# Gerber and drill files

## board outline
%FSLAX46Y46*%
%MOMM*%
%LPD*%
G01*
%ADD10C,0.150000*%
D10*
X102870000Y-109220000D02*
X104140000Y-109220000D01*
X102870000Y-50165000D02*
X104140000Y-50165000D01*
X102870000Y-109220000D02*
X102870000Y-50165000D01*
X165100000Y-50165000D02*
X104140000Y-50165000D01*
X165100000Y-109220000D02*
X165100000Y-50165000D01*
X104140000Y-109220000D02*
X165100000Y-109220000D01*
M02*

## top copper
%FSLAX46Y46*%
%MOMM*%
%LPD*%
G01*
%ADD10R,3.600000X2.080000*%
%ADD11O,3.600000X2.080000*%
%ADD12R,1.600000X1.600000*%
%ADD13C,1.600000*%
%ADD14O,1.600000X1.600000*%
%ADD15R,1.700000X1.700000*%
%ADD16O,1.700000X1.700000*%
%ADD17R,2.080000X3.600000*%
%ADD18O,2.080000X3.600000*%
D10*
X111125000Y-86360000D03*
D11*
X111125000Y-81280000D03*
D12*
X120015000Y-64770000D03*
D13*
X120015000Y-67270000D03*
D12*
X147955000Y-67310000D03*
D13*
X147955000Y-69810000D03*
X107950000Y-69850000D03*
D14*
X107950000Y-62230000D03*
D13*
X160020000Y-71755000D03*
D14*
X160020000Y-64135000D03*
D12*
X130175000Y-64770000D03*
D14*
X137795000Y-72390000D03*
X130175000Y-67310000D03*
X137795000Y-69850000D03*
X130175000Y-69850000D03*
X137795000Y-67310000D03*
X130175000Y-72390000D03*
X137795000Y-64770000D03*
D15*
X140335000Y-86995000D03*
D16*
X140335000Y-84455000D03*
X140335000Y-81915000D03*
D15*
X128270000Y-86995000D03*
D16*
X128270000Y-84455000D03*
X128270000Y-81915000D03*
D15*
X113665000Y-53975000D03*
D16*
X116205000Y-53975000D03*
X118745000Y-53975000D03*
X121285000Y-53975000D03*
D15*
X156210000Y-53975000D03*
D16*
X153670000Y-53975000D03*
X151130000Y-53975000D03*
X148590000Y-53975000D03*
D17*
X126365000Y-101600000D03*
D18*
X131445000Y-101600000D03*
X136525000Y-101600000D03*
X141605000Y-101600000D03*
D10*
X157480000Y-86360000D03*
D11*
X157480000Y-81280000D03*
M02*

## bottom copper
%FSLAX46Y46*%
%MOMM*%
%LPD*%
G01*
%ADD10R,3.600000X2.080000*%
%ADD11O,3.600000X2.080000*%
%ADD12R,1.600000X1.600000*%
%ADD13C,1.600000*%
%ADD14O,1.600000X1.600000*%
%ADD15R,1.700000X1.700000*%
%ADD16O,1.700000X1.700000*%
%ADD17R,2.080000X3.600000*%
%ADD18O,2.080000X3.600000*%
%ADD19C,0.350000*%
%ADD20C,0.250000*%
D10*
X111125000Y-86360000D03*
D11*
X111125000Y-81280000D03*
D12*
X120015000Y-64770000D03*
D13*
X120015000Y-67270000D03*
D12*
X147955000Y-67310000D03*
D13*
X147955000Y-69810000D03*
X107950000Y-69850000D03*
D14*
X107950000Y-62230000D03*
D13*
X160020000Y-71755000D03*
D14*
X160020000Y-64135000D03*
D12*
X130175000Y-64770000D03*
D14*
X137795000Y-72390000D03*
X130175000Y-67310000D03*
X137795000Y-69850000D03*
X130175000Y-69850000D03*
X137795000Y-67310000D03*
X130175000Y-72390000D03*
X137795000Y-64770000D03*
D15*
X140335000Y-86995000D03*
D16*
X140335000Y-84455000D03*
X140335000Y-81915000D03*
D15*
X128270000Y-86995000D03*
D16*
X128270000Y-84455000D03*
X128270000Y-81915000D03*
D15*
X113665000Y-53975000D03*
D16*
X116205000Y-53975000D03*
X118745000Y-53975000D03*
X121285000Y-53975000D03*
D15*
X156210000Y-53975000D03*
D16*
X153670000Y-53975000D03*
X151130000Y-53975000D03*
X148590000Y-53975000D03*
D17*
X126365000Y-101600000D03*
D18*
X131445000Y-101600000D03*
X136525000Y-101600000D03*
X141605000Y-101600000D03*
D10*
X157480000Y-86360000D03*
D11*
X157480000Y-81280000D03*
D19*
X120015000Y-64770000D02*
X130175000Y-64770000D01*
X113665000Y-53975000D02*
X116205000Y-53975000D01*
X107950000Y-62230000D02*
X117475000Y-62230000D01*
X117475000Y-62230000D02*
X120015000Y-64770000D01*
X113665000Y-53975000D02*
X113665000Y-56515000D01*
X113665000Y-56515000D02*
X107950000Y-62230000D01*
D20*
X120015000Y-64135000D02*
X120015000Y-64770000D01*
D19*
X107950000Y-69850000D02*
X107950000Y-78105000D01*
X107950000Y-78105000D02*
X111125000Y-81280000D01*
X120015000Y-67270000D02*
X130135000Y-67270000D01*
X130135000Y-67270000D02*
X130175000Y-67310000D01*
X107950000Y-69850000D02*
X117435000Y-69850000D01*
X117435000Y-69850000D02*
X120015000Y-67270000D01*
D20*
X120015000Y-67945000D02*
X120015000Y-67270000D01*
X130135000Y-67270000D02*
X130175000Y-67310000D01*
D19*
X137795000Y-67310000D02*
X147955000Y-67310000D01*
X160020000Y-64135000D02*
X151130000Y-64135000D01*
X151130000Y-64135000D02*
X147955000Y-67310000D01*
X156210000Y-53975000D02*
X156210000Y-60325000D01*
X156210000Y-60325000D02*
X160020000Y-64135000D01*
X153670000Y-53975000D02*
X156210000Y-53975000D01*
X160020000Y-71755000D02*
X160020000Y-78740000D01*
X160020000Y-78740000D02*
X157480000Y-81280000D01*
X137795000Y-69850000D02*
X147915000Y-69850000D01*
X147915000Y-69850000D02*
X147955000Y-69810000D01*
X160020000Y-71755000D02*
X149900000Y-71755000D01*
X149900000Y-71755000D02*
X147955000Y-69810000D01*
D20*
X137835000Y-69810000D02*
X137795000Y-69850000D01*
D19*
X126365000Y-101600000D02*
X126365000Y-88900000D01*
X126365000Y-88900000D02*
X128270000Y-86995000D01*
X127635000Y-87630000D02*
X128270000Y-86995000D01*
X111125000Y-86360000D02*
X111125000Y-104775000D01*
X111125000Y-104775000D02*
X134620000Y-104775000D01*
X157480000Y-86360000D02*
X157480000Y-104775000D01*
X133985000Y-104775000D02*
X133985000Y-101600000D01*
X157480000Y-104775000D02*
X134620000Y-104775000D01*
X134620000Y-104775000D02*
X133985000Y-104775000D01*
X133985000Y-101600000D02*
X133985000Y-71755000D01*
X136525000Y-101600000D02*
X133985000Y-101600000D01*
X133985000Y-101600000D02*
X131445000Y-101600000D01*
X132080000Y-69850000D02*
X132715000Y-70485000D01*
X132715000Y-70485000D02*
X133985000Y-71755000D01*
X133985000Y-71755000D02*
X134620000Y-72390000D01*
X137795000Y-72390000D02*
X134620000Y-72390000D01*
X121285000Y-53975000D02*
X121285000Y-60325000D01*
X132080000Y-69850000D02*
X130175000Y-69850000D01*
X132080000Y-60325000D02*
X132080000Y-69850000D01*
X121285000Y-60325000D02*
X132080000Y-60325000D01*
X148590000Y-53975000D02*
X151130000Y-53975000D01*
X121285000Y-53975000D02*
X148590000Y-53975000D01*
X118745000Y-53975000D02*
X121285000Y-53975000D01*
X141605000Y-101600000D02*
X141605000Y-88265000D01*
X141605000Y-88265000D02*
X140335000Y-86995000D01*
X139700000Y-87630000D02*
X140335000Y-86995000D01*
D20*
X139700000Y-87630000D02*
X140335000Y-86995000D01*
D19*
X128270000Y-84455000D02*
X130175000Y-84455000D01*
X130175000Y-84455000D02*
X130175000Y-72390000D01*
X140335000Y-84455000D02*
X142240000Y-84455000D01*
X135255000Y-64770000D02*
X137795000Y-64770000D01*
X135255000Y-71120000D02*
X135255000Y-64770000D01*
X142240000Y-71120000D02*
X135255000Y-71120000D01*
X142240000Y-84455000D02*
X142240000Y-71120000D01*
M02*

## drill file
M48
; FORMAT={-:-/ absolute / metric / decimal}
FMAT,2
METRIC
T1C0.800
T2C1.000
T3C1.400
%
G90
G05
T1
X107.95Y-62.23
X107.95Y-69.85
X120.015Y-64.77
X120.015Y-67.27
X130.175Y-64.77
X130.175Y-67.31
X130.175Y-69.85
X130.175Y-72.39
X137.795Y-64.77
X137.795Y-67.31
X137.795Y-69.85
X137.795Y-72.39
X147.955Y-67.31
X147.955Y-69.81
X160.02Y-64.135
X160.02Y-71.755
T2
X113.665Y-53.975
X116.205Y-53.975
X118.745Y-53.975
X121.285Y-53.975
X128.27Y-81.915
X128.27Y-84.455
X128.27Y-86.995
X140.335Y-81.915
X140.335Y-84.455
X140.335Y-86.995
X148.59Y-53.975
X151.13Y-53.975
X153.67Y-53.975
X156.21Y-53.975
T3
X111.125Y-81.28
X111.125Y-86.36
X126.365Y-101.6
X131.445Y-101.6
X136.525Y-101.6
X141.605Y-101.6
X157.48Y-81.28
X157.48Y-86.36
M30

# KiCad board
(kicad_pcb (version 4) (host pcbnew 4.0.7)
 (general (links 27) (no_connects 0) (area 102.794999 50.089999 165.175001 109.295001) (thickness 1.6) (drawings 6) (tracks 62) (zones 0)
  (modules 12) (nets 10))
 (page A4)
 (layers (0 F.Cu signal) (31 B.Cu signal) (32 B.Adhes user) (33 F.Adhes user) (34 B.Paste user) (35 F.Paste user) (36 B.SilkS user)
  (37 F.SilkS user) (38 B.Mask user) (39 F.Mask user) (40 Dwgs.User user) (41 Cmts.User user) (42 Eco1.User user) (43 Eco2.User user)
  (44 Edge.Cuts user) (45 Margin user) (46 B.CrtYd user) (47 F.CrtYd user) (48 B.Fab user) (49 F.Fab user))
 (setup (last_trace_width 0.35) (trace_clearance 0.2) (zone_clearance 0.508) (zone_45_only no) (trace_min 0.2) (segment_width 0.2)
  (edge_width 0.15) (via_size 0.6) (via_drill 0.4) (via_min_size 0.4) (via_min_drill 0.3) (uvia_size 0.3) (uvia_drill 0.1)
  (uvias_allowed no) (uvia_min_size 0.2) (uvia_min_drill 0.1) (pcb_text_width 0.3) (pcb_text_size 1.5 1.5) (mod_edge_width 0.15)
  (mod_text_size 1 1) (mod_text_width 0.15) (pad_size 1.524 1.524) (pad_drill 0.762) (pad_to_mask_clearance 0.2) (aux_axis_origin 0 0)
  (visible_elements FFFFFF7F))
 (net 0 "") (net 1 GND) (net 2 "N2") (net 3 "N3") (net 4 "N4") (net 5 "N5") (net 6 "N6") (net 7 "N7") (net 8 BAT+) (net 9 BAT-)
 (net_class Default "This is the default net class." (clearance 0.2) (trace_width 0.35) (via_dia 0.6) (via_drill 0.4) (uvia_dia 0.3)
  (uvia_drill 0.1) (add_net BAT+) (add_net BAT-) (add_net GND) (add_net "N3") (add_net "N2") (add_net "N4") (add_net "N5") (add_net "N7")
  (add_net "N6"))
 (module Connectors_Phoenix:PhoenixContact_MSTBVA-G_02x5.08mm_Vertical (layer F.Cu) (at 111.125 86.36 90)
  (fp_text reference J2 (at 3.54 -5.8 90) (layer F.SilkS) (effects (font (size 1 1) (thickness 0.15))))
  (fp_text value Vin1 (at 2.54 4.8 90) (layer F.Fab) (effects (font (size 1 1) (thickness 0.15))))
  (pad 1 thru_hole rect (at 0 0 90) (size 2.08 3.6) (drill 1.4) (layers *.Cu *.Mask) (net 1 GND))
  (pad 2 thru_hole oval (at 5.08 0 90) (size 2.08 3.6) (drill 1.4) (layers *.Cu *.Mask) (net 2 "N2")))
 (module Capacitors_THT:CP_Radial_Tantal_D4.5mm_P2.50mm (layer F.Cu) (at 120.015 64.77 270)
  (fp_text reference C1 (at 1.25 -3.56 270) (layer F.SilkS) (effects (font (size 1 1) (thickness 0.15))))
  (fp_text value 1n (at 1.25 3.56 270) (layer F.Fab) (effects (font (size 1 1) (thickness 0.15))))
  (pad 1 thru_hole rect (at 0 0 270) (size 1.6 1.6) (drill 0.8) (layers *.Cu *.Mask) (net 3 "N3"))
  (pad 2 thru_hole circle (at 2.5 0 270) (size 1.6 1.6) (drill 0.8) (layers *.Cu *.Mask) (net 2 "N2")))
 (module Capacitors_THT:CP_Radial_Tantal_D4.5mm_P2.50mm (layer F.Cu) (at 147.955 67.31 270)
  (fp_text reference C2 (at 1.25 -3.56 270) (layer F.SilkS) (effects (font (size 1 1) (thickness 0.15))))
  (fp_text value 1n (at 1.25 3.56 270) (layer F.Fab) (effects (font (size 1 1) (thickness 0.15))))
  (pad 1 thru_hole rect (at 0 0 270) (size 1.6 1.6) (drill 0.8) (layers *.Cu *.Mask) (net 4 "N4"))
  (pad 2 thru_hole circle (at 2.5 0 270) (size 1.6 1.6) (drill 0.8) (layers *.Cu *.Mask) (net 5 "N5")))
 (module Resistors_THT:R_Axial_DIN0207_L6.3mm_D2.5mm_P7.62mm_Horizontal (layer F.Cu) (at 107.95 69.85 90)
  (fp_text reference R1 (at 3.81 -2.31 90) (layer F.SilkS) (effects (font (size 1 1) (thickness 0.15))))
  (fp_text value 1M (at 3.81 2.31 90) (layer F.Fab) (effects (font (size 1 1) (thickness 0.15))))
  (pad 1 thru_hole circle (at 0 0 90) (size 1.6 1.6) (drill 0.8) (layers *.Cu *.Mask) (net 2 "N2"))
  (pad 2 thru_hole oval (at 7.62 0 90) (size 1.6 1.6) (drill 0.8) (layers *.Cu *.Mask) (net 3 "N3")))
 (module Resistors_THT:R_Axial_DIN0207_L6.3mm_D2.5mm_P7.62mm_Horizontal (layer F.Cu) (at 160.02 71.755 90)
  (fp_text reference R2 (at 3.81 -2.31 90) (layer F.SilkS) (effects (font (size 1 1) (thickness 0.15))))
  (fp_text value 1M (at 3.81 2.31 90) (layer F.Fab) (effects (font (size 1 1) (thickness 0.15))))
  (pad 1 thru_hole circle (at 0 0 90) (size 1.6 1.6) (drill 0.8) (layers *.Cu *.Mask) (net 5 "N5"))
  (pad 2 thru_hole oval (at 7.62 0 90) (size 1.6 1.6) (drill 0.8) (layers *.Cu *.Mask) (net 4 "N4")))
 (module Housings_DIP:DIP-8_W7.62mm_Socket (layer F.Cu) (at 130.175 64.77)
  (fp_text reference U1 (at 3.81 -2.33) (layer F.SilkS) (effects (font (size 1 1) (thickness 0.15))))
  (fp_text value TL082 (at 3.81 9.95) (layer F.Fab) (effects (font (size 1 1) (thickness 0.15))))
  (pad 1 thru_hole rect (at 0 0) (size 1.6 1.6) (drill 0.8) (layers *.Cu *.Mask) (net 3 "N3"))
  (pad 5 thru_hole oval (at 7.62 7.62) (size 1.6 1.6) (drill 0.8) (layers *.Cu *.Mask) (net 1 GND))
  (pad 2 thru_hole oval (at 0 2.54) (size 1.6 1.6) (drill 0.8) (layers *.Cu *.Mask) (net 2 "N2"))
  (pad 6 thru_hole oval (at 7.62 5.08) (size 1.6 1.6) (drill 0.8) (layers *.Cu *.Mask) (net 5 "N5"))
  (pad 3 thru_hole oval (at 0 5.08) (size 1.6 1.6) (drill 0.8) (layers *.Cu *.Mask) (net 1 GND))
  (pad 7 thru_hole oval (at 7.62 2.54) (size 1.6 1.6) (drill 0.8) (layers *.Cu *.Mask) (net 4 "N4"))
  (pad 4 thru_hole oval (at 0 7.62) (size 1.6 1.6) (drill 0.8) (layers *.Cu *.Mask) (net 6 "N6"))
  (pad 8 thru_hole oval (at 7.62 0) (size 1.6 1.6) (drill 0.8) (layers *.Cu *.Mask) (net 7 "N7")))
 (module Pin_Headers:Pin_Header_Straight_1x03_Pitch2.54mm (layer F.Cu) (at 140.335 86.995 180)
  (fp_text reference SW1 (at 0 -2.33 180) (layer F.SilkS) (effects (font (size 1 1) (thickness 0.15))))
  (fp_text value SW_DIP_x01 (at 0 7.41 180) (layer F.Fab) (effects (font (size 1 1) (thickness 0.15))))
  (pad 1 thru_hole rect (at 0 0 180) (size 1.7 1.7) (drill 1) (layers *.Cu *.Mask) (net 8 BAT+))
  (pad 2 thru_hole oval (at 0 2.54 180) (size 1.7 1.7) (drill 1) (layers *.Cu *.Mask) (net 7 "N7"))
  (pad 3 thru_hole oval (at 0 5.08 180) (size 1.7 1.7) (drill 1) (layers *.Cu *.Mask)))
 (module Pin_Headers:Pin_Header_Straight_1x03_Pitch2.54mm (layer F.Cu) (at 128.27 86.995 180)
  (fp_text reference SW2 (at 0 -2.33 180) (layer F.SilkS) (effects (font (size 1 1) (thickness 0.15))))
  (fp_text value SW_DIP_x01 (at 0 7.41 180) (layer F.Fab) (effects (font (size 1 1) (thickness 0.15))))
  (pad 1 thru_hole rect (at 0 0 180) (size 1.7 1.7) (drill 1) (layers *.Cu *.Mask) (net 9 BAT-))
  (pad 2 thru_hole oval (at 0 2.54 180) (size 1.7 1.7) (drill 1) (layers *.Cu *.Mask) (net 6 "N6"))
  (pad 3 thru_hole oval (at 0 5.08 180) (size 1.7 1.7) (drill 1) (layers *.Cu *.Mask)))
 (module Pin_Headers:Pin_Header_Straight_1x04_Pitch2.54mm (layer F.Cu) (at 113.665 53.975 90)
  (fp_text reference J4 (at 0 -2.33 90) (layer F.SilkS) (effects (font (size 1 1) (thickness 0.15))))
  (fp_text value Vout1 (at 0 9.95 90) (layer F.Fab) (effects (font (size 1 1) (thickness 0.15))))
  (pad 1 thru_hole rect (at 0 0 90) (size 1.7 1.7) (drill 1) (layers *.Cu *.Mask) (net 3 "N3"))
  (pad 2 thru_hole oval (at 0 2.54 90) (size 1.7 1.7) (drill 1) (layers *.Cu *.Mask) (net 3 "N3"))
  (pad 3 thru_hole oval (at 0 5.08 90) (size 1.7 1.7) (drill 1) (layers *.Cu *.Mask) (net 1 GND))
  (pad 4 thru_hole oval (at 0 7.62 90) (size 1.7 1.7) (drill 1) (layers *.Cu *.Mask) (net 1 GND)))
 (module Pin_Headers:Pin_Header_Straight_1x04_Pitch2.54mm (layer F.Cu) (at 156.21 53.975 270)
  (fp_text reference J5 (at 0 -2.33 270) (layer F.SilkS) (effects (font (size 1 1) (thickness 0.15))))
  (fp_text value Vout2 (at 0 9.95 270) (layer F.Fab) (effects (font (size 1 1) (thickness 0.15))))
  (pad 1 thru_hole rect (at 0 0 270) (size 1.7 1.7) (drill 1) (layers *.Cu *.Mask) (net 4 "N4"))
  (pad 2 thru_hole oval (at 0 2.54 270) (size 1.7 1.7) (drill 1) (layers *.Cu *.Mask) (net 4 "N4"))
  (pad 3 thru_hole oval (at 0 5.08 270) (size 1.7 1.7) (drill 1) (layers *.Cu *.Mask) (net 1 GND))
  (pad 4 thru_hole oval (at 0 7.62 270) (size 1.7 1.7) (drill 1) (layers *.Cu *.Mask) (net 1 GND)))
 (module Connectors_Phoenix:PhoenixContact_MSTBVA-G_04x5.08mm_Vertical (layer F.Cu) (at 126.365 101.6)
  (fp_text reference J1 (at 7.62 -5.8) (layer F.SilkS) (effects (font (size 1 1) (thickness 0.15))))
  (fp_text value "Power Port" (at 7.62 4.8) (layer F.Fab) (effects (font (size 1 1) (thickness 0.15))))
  (pad 1 thru_hole rect (at 0 0) (size 2.08 3.6) (drill 1.4) (layers *.Cu *.Mask) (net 9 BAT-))
  (pad 2 thru_hole oval (at 5.08 0) (size 2.08 3.6) (drill 1.4) (layers *.Cu *.Mask) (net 1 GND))
  (pad 3 thru_hole oval (at 10.16 0) (size 2.08 3.6) (drill 1.4) (layers *.Cu *.Mask) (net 1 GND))
  (pad 4 thru_hole oval (at 15.24 0) (size 2.08 3.6) (drill 1.4) (layers *.Cu *.Mask) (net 8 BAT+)))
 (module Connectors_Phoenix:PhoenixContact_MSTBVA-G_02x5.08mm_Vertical (layer F.Cu) (at 157.48 86.36 90)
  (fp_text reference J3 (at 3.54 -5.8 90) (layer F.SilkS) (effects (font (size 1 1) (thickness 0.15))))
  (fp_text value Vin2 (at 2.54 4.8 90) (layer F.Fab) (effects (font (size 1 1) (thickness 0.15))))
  (pad 1 thru_hole rect (at 0 0 90) (size 2.08 3.6) (drill 1.4) (layers *.Cu *.Mask) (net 1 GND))
  (pad 2 thru_hole oval (at 5.08 0 90) (size 2.08 3.6) (drill 1.4) (layers *.Cu *.Mask) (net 5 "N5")))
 (gr_line (start 102.87 109.22) (end 104.14 109.22) (angle 90) (layer Edge.Cuts) (width 0.15))
 (gr_line (start 102.87 50.165) (end 104.14 50.165) (angle 90) (layer Edge.Cuts) (width 0.15))
 (gr_line (start 102.87 109.22) (end 102.87 50.165) (angle 90) (layer Edge.Cuts) (width 0.15))
 (gr_line (start 165.1 50.165) (end 104.14 50.165) (angle 90) (layer Edge.Cuts) (width 0.15))
 (gr_line (start 165.1 109.22) (end 165.1 50.165) (angle 90) (layer Edge.Cuts) (width 0.15))
 (gr_line (start 104.14 109.22) (end 165.1 109.22) (angle 90) (layer Edge.Cuts) (width 0.15))
 (segment (start 120.015 64.77) (end 130.175 64.77) (width 0.35) (layer B.Cu) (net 3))
 (segment (start 113.665 53.975) (end 116.205 53.975) (width 0.35) (layer B.Cu) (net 3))
 (segment (start 107.95 62.23) (end 117.475 62.23) (width 0.35) (layer B.Cu) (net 3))
 (segment (start 117.475 62.23) (end 120.015 64.77) (width 0.35) (layer B.Cu) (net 3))
 (segment (start 113.665 53.975) (end 113.665 56.515) (width 0.35) (layer B.Cu) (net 3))
 (segment (start 113.665 56.515) (end 107.95 62.23) (width 0.35) (layer B.Cu) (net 3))
 (segment (start 120.015 64.135) (end 120.015 64.77) (width 0.25) (layer B.Cu) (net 3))
 (segment (start 107.95 69.85) (end 107.95 78.105) (width 0.35) (layer B.Cu) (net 2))
 (segment (start 107.95 78.105) (end 111.125 81.28) (width 0.35) (layer B.Cu) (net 2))
 (segment (start 120.015 67.27) (end 130.135 67.27) (width 0.35) (layer B.Cu) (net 2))
 (segment (start 130.135 67.27) (end 130.175 67.31) (width 0.35) (layer B.Cu) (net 2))
 (segment (start 107.95 69.85) (end 117.435 69.85) (width 0.35) (layer B.Cu) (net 2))
 (segment (start 117.435 69.85) (end 120.015 67.27) (width 0.35) (layer B.Cu) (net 2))
 (segment (start 120.015 67.945) (end 120.015 67.27) (width 0.25) (layer B.Cu) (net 2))
 (segment (start 130.135 67.27) (end 130.175 67.31) (width 0.25) (layer B.Cu) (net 2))
 (segment (start 137.795 67.31) (end 147.955 67.31) (width 0.35) (layer B.Cu) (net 4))
 (segment (start 160.02 64.135) (end 151.13 64.135) (width 0.35) (layer B.Cu) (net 4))
 (segment (start 151.13 64.135) (end 147.955 67.31) (width 0.35) (layer B.Cu) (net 4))
 (segment (start 156.21 53.975) (end 156.21 60.325) (width 0.35) (layer B.Cu) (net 4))
 (segment (start 156.21 60.325) (end 160.02 64.135) (width 0.35) (layer B.Cu) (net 4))
 (segment (start 153.67 53.975) (end 156.21 53.975) (width 0.35) (layer B.Cu) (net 4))
 (segment (start 160.02 71.755) (end 160.02 78.74) (width 0.35) (layer B.Cu) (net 5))
 (segment (start 160.02 78.74) (end 157.48 81.28) (width 0.35) (layer B.Cu) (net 5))
 (segment (start 137.795 69.85) (end 147.915 69.85) (width 0.35) (layer B.Cu) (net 5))
 (segment (start 147.915 69.85) (end 147.955 69.81) (width 0.35) (layer B.Cu) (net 5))
 (segment (start 160.02 71.755) (end 149.9 71.755) (width 0.35) (layer B.Cu) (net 5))
 (segment (start 149.9 71.755) (end 147.955 69.81) (width 0.35) (layer B.Cu) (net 5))
 (segment (start 137.835 69.81) (end 137.795 69.85) (width 0.25) (layer B.Cu) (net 5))
 (segment (start 126.365 101.6) (end 126.365 88.9) (width 0.35) (layer B.Cu) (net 9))
 (segment (start 126.365 88.9) (end 128.27 86.995) (width 0.35) (layer B.Cu) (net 9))
 (segment (start 127.635 87.63) (end 128.27 86.995) (width 0.35) (layer B.Cu) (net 9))
 (segment (start 111.125 86.36) (end 111.125 104.775) (width 0.35) (layer B.Cu) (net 1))
 (segment (start 111.125 104.775) (end 134.62 104.775) (width 0.35) (layer B.Cu) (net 1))
 (segment (start 157.48 86.36) (end 157.48 104.775) (width 0.35) (layer B.Cu) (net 1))
 (segment (start 133.985 104.775) (end 133.985 101.6) (width 0.35) (layer B.Cu) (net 1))
 (segment (start 157.48 104.775) (end 134.62 104.775) (width 0.35) (layer B.Cu) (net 1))
 (segment (start 134.62 104.775) (end 133.985 104.775) (width 0.35) (layer B.Cu) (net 1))
 (segment (start 133.985 101.6) (end 133.985 71.755) (width 0.35) (layer B.Cu) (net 1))
 (segment (start 136.525 101.6) (end 133.985 101.6) (width 0.35) (layer B.Cu) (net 1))
 (segment (start 133.985 101.6) (end 131.445 101.6) (width 0.35) (layer B.Cu) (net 1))
 (segment (start 132.08 69.85) (end 132.715 70.485) (width 0.35) (layer B.Cu) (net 1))
 (segment (start 132.715 70.485) (end 133.985 71.755) (width 0.35) (layer B.Cu) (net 1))
 (segment (start 133.985 71.755) (end 134.62 72.39) (width 0.35) (layer B.Cu) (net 1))
 (segment (start 137.795 72.39) (end 134.62 72.39) (width 0.35) (layer B.Cu) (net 1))
 (segment (start 121.285 53.975) (end 121.285 60.325) (width 0.35) (layer B.Cu) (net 1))
 (segment (start 132.08 69.85) (end 130.175 69.85) (width 0.35) (layer B.Cu) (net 1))
 (segment (start 132.08 60.325) (end 132.08 69.85) (width 0.35) (layer B.Cu) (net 1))
 (segment (start 121.285 60.325) (end 132.08 60.325) (width 0.35) (layer B.Cu) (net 1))
 (segment (start 148.59 53.975) (end 151.13 53.975) (width 0.35) (layer B.Cu) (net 1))
 (segment (start 121.285 53.975) (end 148.59 53.975) (width 0.35) (layer B.Cu) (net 1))
 (segment (start 118.745 53.975) (end 121.285 53.975) (width 0.35) (layer B.Cu) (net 1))
 (segment (start 141.605 101.6) (end 141.605 88.265) (width 0.35) (layer B.Cu) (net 8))
 (segment (start 141.605 88.265) (end 140.335 86.995) (width 0.35) (layer B.Cu) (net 8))
 (segment (start 139.7 87.63) (end 140.335 86.995) (width 0.35) (layer B.Cu) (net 8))
 (segment (start 139.7 87.63) (end 140.335 86.995) (width 0.25) (layer B.Cu) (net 8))
 (segment (start 128.27 84.455) (end 130.175 84.455) (width 0.35) (layer B.Cu) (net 6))
 (segment (start 130.175 84.455) (end 130.175 72.39) (width 0.35) (layer B.Cu) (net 6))
 (segment (start 140.335 84.455) (end 142.24 84.455) (width 0.35) (layer B.Cu) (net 7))
 (segment (start 135.255 64.77) (end 137.795 64.77) (width 0.35) (layer B.Cu) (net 7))
 (segment (start 135.255 71.12) (end 135.255 64.77) (width 0.35) (layer B.Cu) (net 7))
 (segment (start 142.24 71.12) (end 135.255 71.12) (width 0.35) (layer B.Cu) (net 7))
 (segment (start 142.24 84.455) (end 142.24 71.12) (width 0.35) (layer B.Cu) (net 7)))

